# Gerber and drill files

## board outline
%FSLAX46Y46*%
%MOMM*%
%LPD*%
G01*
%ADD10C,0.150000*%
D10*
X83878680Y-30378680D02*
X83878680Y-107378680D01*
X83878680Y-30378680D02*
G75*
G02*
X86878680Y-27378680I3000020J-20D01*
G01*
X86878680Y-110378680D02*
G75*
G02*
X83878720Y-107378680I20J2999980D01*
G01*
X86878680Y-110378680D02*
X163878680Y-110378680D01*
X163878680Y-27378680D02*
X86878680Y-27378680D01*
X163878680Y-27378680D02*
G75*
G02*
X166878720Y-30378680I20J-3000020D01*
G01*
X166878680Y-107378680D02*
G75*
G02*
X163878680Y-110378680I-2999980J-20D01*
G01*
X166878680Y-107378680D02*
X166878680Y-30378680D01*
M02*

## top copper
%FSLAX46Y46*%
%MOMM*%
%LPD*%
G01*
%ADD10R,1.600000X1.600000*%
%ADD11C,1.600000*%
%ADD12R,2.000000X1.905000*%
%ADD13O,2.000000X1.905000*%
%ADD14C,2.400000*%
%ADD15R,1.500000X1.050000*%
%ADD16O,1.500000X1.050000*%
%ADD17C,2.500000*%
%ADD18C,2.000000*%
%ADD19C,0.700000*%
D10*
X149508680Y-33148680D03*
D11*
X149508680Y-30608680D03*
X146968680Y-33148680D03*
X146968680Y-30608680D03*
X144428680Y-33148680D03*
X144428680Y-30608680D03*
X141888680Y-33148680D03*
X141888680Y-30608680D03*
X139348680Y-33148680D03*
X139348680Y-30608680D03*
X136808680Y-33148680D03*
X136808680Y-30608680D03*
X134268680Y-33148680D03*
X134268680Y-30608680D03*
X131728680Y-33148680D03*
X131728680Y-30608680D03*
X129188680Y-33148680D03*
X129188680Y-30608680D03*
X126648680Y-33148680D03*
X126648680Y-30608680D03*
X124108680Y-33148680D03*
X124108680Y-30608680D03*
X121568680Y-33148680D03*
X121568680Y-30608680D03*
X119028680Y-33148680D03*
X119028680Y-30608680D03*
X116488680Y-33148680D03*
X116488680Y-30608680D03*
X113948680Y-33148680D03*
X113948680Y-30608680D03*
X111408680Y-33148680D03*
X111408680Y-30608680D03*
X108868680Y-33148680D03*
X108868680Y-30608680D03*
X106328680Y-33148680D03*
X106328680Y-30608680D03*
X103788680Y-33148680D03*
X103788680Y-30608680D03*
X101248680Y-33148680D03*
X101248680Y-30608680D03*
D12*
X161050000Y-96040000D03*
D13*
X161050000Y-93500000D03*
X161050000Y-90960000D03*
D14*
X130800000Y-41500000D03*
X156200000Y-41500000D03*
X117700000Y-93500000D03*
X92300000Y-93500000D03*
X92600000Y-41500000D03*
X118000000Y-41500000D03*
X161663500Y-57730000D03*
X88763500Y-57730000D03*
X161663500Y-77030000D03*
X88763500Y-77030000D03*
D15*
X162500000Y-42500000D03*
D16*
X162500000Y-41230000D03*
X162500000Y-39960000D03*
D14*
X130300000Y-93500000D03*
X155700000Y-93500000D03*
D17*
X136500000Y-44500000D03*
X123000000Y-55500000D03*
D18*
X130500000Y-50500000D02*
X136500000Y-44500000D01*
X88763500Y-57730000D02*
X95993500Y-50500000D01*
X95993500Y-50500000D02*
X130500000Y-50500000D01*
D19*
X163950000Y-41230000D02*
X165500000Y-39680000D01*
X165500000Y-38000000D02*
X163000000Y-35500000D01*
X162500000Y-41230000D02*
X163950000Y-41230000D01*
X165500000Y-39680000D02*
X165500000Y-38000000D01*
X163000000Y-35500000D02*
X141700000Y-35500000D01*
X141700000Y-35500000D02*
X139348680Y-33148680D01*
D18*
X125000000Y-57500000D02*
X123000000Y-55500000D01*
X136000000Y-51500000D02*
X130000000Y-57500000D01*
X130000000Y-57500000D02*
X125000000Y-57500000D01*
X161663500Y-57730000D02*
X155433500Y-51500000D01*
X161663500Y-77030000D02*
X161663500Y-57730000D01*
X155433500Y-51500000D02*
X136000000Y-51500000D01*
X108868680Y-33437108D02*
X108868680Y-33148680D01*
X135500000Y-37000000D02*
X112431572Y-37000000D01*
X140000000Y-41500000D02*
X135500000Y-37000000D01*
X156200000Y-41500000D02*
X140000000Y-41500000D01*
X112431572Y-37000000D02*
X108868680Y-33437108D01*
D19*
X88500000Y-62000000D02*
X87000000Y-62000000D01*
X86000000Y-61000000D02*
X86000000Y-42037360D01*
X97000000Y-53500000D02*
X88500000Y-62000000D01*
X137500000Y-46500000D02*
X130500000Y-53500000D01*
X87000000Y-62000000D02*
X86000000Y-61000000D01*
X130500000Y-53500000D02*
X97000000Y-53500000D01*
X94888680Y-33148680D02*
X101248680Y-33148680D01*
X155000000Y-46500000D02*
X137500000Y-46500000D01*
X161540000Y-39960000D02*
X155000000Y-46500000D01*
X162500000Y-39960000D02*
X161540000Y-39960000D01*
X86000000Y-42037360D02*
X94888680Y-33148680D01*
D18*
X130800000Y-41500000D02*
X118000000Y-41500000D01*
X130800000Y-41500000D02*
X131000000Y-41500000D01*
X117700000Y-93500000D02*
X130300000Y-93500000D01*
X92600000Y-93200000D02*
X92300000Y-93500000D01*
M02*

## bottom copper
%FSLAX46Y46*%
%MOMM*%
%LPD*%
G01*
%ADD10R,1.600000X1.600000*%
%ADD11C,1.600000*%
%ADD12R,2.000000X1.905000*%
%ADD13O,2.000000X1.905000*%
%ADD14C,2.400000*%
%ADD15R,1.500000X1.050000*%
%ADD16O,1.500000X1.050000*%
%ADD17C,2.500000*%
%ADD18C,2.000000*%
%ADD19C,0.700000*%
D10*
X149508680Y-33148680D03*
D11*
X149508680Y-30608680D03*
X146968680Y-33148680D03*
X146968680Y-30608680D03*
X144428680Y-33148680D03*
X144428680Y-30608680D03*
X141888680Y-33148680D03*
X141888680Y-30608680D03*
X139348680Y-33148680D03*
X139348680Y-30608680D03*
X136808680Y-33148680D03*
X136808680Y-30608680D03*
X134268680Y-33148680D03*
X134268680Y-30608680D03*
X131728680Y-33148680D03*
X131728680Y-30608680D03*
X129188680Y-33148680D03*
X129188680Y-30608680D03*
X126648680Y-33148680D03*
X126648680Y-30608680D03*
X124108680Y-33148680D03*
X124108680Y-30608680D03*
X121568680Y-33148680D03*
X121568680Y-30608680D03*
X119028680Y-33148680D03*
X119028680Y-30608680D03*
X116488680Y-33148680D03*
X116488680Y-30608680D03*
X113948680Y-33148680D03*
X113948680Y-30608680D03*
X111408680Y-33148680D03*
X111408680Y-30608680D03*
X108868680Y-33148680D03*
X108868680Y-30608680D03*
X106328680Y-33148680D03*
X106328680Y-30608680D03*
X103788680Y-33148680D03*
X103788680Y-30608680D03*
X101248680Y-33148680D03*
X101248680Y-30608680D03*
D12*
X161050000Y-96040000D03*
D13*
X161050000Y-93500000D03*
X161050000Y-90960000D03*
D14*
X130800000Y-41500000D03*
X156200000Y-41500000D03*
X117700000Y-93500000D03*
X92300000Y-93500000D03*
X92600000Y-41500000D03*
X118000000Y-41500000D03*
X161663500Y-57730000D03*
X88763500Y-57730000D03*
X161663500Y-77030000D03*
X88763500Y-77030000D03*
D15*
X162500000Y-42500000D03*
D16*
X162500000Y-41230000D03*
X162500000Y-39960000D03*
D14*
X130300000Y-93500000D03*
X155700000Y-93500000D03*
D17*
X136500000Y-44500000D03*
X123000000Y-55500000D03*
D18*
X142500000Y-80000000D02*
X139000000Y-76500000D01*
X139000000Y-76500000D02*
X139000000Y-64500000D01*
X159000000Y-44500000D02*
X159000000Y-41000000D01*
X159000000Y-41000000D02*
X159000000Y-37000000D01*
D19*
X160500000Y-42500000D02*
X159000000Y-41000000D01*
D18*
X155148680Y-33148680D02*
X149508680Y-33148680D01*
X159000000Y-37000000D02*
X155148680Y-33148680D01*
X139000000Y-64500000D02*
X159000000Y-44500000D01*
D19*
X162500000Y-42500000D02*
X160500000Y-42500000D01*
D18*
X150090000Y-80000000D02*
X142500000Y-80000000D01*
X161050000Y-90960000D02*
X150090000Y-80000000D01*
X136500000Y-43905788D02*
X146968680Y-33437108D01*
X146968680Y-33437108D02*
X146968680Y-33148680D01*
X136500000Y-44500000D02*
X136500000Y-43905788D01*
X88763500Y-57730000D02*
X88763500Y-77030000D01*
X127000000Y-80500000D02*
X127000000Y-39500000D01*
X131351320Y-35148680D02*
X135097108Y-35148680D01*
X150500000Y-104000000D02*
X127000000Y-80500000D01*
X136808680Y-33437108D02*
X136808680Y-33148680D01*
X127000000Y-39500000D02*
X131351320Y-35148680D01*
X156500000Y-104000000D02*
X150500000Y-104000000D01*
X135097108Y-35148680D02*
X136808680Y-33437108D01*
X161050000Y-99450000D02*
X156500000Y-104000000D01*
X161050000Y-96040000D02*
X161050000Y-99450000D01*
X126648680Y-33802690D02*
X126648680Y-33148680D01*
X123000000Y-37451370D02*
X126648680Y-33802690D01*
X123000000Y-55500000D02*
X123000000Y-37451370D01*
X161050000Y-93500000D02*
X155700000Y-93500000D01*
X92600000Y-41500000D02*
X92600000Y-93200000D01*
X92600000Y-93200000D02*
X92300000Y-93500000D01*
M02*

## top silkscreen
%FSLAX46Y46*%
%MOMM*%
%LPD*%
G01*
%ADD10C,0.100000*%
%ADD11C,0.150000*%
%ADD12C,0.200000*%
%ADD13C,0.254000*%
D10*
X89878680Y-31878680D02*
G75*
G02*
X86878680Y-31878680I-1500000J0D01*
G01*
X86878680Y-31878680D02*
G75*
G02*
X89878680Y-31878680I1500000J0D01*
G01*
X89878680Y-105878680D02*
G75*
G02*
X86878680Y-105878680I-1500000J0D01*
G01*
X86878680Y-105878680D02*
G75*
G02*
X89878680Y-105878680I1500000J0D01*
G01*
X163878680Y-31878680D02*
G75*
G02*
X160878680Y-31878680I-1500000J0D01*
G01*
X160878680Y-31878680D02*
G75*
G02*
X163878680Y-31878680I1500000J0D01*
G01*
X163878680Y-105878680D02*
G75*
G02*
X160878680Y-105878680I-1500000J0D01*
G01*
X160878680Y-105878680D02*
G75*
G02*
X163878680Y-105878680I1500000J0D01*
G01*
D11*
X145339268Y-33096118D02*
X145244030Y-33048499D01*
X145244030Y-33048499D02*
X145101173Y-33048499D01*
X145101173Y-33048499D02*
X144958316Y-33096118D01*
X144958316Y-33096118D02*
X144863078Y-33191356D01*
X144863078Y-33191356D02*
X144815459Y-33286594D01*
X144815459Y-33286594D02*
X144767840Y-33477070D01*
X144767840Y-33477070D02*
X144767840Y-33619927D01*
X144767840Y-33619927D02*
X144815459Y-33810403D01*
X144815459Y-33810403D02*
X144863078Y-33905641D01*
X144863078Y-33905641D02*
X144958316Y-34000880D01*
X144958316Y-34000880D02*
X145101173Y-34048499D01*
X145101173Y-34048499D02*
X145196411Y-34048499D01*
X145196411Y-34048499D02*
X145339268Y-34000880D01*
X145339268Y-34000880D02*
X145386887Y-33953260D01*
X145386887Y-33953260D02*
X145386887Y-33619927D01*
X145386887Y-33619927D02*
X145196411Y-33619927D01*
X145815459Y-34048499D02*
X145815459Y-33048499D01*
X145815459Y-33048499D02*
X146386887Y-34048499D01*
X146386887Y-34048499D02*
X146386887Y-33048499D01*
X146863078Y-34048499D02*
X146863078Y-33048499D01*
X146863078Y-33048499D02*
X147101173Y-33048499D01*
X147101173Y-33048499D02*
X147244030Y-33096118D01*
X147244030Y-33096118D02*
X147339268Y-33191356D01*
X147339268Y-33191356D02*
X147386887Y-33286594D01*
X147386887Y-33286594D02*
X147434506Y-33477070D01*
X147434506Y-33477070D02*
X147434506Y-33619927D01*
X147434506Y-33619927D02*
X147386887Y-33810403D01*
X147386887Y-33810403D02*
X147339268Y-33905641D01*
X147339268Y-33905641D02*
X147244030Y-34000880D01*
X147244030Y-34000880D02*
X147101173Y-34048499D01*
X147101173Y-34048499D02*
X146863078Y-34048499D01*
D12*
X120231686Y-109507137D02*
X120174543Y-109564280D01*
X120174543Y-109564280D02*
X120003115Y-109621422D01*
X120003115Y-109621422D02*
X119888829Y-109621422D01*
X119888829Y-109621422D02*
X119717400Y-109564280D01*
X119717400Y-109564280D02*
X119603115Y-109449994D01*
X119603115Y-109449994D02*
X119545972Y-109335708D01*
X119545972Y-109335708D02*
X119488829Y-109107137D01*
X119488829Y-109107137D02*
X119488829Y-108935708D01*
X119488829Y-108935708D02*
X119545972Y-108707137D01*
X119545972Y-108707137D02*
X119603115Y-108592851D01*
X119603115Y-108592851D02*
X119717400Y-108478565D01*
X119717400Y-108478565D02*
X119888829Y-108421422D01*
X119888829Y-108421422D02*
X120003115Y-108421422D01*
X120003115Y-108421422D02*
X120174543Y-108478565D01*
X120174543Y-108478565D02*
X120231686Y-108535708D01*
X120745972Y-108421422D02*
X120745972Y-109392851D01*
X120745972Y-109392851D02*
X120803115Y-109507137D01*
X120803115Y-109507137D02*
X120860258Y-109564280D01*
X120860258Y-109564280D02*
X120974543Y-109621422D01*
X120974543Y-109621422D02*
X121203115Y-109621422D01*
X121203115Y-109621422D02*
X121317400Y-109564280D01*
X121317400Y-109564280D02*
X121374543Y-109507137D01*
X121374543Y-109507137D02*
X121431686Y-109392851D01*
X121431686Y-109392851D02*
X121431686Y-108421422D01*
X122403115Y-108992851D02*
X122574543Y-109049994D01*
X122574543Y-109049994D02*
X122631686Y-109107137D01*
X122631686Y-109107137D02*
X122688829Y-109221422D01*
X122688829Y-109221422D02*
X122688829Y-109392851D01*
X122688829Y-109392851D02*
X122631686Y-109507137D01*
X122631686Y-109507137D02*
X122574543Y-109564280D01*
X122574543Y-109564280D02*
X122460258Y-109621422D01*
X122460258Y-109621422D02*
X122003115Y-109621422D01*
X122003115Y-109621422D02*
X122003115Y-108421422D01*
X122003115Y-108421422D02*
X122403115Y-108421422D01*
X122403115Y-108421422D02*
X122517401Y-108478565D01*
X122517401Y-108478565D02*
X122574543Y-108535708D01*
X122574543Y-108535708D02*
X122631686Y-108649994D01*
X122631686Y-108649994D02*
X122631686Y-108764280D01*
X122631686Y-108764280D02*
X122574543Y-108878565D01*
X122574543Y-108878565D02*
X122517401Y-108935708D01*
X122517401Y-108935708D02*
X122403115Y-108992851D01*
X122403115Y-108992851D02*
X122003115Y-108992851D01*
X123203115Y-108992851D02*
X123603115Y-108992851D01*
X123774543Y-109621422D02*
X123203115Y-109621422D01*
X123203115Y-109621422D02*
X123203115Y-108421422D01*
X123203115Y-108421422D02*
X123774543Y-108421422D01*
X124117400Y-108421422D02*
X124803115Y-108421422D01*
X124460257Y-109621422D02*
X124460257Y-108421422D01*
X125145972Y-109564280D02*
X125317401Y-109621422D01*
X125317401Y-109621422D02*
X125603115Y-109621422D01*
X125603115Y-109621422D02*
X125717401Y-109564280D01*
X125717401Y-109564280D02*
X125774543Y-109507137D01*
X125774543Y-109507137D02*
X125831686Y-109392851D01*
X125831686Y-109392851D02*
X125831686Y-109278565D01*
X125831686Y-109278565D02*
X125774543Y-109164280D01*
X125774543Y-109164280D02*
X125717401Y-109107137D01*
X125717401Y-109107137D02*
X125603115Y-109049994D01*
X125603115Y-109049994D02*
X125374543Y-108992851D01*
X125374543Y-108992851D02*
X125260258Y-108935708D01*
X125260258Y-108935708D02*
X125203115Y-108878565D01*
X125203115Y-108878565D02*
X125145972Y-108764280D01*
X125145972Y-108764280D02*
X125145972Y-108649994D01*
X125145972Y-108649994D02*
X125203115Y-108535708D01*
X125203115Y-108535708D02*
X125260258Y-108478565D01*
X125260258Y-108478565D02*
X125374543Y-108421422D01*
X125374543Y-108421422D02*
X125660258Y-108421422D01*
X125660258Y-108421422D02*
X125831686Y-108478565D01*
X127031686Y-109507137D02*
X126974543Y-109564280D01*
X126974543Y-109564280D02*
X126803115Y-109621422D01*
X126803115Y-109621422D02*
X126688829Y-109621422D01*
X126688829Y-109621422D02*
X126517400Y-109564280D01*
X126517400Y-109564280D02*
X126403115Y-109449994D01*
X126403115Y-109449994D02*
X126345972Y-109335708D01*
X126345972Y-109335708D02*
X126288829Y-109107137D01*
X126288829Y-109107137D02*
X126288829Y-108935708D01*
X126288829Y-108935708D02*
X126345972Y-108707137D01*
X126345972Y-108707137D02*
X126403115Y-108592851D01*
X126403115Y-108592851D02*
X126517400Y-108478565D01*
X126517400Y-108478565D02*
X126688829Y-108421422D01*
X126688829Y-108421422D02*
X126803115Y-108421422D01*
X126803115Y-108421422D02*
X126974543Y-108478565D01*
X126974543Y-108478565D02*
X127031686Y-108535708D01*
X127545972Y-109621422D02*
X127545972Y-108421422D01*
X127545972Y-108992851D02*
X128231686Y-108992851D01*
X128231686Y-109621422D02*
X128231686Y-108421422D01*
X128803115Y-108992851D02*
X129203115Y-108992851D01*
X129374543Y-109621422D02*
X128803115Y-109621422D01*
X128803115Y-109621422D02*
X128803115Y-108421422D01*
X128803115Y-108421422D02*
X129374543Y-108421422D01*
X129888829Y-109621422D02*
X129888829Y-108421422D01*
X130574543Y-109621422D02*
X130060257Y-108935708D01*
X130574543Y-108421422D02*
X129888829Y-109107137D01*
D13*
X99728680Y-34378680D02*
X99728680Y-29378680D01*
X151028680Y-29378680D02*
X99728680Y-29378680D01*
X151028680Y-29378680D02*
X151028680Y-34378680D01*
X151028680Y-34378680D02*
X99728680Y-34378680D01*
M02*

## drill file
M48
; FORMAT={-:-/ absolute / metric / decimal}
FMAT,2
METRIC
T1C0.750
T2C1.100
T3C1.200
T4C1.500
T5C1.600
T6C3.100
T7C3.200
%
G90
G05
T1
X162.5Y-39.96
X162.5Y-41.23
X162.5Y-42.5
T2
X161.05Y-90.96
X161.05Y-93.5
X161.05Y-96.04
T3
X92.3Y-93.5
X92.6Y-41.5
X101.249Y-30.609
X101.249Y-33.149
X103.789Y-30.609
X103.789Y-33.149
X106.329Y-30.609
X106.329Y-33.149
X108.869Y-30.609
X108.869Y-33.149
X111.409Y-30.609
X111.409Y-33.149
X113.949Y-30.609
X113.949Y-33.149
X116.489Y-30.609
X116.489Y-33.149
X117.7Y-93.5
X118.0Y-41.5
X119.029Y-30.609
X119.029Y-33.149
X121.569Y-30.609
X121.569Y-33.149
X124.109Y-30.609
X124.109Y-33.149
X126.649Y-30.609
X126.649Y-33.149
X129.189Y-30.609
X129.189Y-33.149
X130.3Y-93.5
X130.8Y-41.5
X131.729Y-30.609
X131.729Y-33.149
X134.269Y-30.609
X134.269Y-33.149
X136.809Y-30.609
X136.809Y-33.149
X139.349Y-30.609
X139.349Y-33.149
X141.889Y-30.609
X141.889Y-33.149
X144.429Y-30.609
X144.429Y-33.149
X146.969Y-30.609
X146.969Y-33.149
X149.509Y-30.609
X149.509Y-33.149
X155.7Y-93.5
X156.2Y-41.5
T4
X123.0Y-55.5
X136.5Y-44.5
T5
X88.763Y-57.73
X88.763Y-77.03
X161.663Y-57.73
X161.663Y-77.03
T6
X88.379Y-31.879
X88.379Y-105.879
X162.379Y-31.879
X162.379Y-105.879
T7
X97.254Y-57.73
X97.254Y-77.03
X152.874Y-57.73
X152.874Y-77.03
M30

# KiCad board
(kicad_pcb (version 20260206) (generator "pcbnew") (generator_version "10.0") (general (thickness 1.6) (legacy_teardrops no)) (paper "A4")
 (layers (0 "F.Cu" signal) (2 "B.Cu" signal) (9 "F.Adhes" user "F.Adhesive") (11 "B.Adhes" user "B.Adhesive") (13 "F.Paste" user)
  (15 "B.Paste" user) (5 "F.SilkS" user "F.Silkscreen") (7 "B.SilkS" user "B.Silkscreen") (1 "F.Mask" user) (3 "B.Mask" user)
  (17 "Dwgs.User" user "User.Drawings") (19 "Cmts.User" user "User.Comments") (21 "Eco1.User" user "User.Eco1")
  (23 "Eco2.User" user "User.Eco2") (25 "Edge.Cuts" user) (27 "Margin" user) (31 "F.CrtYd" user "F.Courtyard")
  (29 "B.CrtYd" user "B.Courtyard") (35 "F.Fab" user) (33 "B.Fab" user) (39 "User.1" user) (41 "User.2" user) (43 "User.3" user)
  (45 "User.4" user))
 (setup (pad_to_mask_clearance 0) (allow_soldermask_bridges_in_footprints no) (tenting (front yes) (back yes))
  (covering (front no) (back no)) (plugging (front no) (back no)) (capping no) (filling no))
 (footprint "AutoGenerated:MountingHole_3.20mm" (layer "F.Cu") (at 88.37868 105.87868)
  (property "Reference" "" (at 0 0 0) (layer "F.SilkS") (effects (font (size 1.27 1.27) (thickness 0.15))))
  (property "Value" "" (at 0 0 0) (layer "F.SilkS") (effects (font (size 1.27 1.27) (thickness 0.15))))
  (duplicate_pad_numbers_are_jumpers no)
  (pad "" np_thru_hole circle (at 0 0) (size 3.1 3.1) (drill 3.1) (layers "*.Cu" "*.Mask")))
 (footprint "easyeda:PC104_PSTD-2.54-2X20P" (layer "F.Cu") (at 149.50868 30.60868 -90)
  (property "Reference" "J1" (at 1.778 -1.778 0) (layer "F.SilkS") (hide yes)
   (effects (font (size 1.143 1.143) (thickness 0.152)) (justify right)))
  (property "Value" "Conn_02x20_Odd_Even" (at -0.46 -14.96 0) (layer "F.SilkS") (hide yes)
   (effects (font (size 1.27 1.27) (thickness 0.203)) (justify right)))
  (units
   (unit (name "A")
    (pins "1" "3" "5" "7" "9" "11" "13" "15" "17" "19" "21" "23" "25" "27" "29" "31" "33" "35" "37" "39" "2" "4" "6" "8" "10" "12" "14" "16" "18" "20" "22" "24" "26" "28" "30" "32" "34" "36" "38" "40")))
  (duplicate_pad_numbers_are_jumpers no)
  (fp_line (start 3.77 49.78) (end -1.23 49.78) (stroke (width 0.254) (type solid)) (layer "F.SilkS"))
  (fp_line (start -1.23 -1.52) (end -1.23 49.78) (stroke (width 0.254) (type solid)) (layer "F.SilkS"))
  (fp_line (start -1.23 -1.52) (end 3.77 -1.52) (stroke (width 0.254) (type solid)) (layer "F.SilkS"))
  (fp_line (start 3.77 -1.52) (end 3.77 49.78) (stroke (width 0.254) (type solid)) (layer "F.SilkS"))
  (pad "1" thru_hole rect (at 2.54 0 180) (size 1.6 1.6) (drill 1.2) (layers "*.Cu" "*.Paste" "*.Mask") (remove_unused_layers no)
   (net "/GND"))
  (pad "2" thru_hole circle (at 0 0 180) (size 1.6 1.6) (drill 1.2) (layers "*.Cu" "*.Paste" "*.Mask") (remove_unused_layers no)
   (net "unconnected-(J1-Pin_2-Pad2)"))
  (pad "3" thru_hole circle (at 2.54 2.54 180) (size 1.6 1.6) (drill 1.2) (layers "*.Cu" "*.Paste" "*.Mask") (remove_unused_layers no)
   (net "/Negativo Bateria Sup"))
  (pad "4" thru_hole circle (at 0 2.54 180) (size 1.6 1.6) (drill 1.2) (layers "*.Cu" "*.Paste" "*.Mask") (remove_unused_layers no)
   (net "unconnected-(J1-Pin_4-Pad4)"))
  (pad "5" thru_hole circle (at 2.54 5.08 180) (size 1.6 1.6) (drill 1.2) (layers "*.Cu" "*.Paste" "*.Mask") (remove_unused_layers no)
   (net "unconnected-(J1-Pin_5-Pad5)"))
  (pad "6" thru_hole circle (at 0 5.08 180) (size 1.6 1.6) (drill 1.2) (layers "*.Cu" "*.Paste" "*.Mask") (remove_unused_layers no)
   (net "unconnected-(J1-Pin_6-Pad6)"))
  (pad "7" thru_hole circle (at 2.54 7.62 180) (size 1.6 1.6) (drill 1.2) (layers "*.Cu" "*.Paste" "*.Mask") (remove_unused_layers no)
   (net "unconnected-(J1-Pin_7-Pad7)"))
  (pad "8" thru_hole circle (at 0 7.62 180) (size 1.6 1.6) (drill 1.2) (layers "*.Cu" "*.Paste" "*.Mask") (remove_unused_layers no)
   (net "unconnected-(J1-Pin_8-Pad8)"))
  (pad "9" thru_hole circle (at 2.54 10.16 180) (size 1.6 1.6) (drill 1.2) (layers "*.Cu" "*.Paste" "*.Mask") (remove_unused_layers no)
   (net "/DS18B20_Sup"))
  (pad "10" thru_hole circle (at 0 10.16 180) (size 1.6 1.6) (drill 1.2) (layers "*.Cu" "*.Paste" "*.Mask") (remove_unused_layers no)
   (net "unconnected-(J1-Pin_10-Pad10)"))
  (pad "11" thru_hole circle (at 2.54 12.7 180) (size 1.6 1.6) (drill 1.2) (layers "*.Cu" "*.Paste" "*.Mask") (remove_unused_layers no)
   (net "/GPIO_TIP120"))
  (pad "12" thru_hole circle (at 0 12.7 180) (size 1.6 1.6) (drill 1.2) (layers "*.Cu" "*.Paste" "*.Mask") (remove_unused_layers no)
   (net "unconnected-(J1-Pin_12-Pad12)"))
  (pad "13" thru_hole circle (at 2.54 15.24 180) (size 1.6 1.6) (drill 1.2) (layers "*.Cu" "*.Paste" "*.Mask") (remove_unused_layers no)
   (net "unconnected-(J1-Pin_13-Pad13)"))
  (pad "14" thru_hole circle (at 0 15.24 180) (size 1.6 1.6) (drill 1.2) (layers "*.Cu" "*.Paste" "*.Mask") (remove_unused_layers no)
   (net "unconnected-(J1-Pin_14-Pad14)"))
  (pad "15" thru_hole circle (at 2.54 17.78 180) (size 1.6 1.6) (drill 1.2) (layers "*.Cu" "*.Paste" "*.Mask") (remove_unused_layers no)
   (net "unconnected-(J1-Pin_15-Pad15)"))
  (pad "16" thru_hole circle (at 0 17.78 180) (size 1.6 1.6) (drill 1.2) (layers "*.Cu" "*.Paste" "*.Mask") (remove_unused_layers no)
   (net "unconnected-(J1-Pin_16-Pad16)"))
  (pad "17" thru_hole circle (at 2.54 20.32 180) (size 1.6 1.6) (drill 1.2) (layers "*.Cu" "*.Paste" "*.Mask") (remove_unused_layers no)
   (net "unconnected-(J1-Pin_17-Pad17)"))
  (pad "18" thru_hole circle (at 0 20.32 180) (size 1.6 1.6) (drill 1.2) (layers "*.Cu" "*.Paste" "*.Mask") (remove_unused_layers no)
   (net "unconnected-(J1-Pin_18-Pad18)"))
  (pad "19" thru_hole circle (at 2.54 22.86 180) (size 1.6 1.6) (drill 1.2) (layers "*.Cu" "*.Paste" "*.Mask") (remove_unused_layers no)
   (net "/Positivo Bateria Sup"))
  (pad "20" thru_hole circle (at 0 22.86 180) (size 1.6 1.6) (drill 1.2) (layers "*.Cu" "*.Paste" "*.Mask") (remove_unused_layers no)
   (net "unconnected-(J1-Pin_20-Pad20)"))
  (pad "21" thru_hole circle (at 2.54 25.4 180) (size 1.6 1.6) (drill 1.2) (layers "*.Cu" "*.Paste" "*.Mask") (remove_unused_layers no)
   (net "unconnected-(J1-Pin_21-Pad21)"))
  (pad "22" thru_hole circle (at 0 25.4 180) (size 1.6 1.6) (drill 1.2) (layers "*.Cu" "*.Paste" "*.Mask") (remove_unused_layers no)
   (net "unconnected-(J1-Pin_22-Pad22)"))
  (pad "23" thru_hole circle (at 2.54 27.94 180) (size 1.6 1.6) (drill 1.2) (layers "*.Cu" "*.Paste" "*.Mask") (remove_unused_layers no)
   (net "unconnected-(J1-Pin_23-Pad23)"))
  (pad "24" thru_hole circle (at 0 27.94 180) (size 1.6 1.6) (drill 1.2) (layers "*.Cu" "*.Paste" "*.Mask") (remove_unused_layers no)
   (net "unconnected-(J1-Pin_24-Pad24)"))
  (pad "25" thru_hole circle (at 2.54 30.48 180) (size 1.6 1.6) (drill 1.2) (layers "*.Cu" "*.Paste" "*.Mask") (remove_unused_layers no)
   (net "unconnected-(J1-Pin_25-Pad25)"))
  (pad "26" thru_hole circle (at 0 30.48 180) (size 1.6 1.6) (drill 1.2) (layers "*.Cu" "*.Paste" "*.Mask") (remove_unused_layers no)
   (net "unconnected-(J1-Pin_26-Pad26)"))
  (pad "27" thru_hole circle (at 2.54 33.02 180) (size 1.6 1.6) (drill 1.2) (layers "*.Cu" "*.Paste" "*.Mask") (remove_unused_layers no)
   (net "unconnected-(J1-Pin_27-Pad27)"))
  (pad "28" thru_hole circle (at 0 33.02 180) (size 1.6 1.6) (drill 1.2) (layers "*.Cu" "*.Paste" "*.Mask") (remove_unused_layers no)
   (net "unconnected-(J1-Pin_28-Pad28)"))
  (pad "29" thru_hole circle (at 2.54 35.56 180) (size 1.6 1.6) (drill 1.2) (layers "*.Cu" "*.Paste" "*.Mask") (remove_unused_layers no)
   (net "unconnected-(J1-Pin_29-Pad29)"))
  (pad "30" thru_hole circle (at 0 35.56 180) (size 1.6 1.6) (drill 1.2) (layers "*.Cu" "*.Paste" "*.Mask") (remove_unused_layers no)
   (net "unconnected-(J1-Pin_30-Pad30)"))
  (pad "31" thru_hole circle (at 2.54 38.1 180) (size 1.6 1.6) (drill 1.2) (layers "*.Cu" "*.Paste" "*.Mask") (remove_unused_layers no)
   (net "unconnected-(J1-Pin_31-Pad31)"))
  (pad "32" thru_hole circle (at 0 38.1 180) (size 1.6 1.6) (drill 1.2) (layers "*.Cu" "*.Paste" "*.Mask") (remove_unused_layers no)
   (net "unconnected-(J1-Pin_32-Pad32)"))
  (pad "33" thru_hole circle (at 2.54 40.64 180) (size 1.6 1.6) (drill 1.2) (layers "*.Cu" "*.Paste" "*.Mask") (remove_unused_layers no)
   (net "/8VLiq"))
  (pad "34" thru_hole circle (at 0 40.64 180) (size 1.6 1.6) (drill 1.2) (layers "*.Cu" "*.Paste" "*.Mask") (remove_unused_layers no)
   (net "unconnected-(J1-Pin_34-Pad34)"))
  (pad "35" thru_hole circle (at 2.54 43.18 180) (size 1.6 1.6) (drill 1.2) (layers "*.Cu" "*.Paste" "*.Mask") (remove_unused_layers no)
   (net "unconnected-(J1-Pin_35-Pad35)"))
  (pad "36" thru_hole circle (at 0 43.18 180) (size 1.6 1.6) (drill 1.2) (layers "*.Cu" "*.Paste" "*.Mask") (remove_unused_layers no)
   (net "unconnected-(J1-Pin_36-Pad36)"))
  (pad "37" thru_hole circle (at 2.54 45.72 180) (size 1.6 1.6) (drill 1.2) (layers "*.Cu" "*.Paste" "*.Mask") (remove_unused_layers no)
   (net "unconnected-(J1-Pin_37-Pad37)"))
  (pad "38" thru_hole circle (at 0 45.72 180) (size 1.6 1.6) (drill 1.2) (layers "*.Cu" "*.Paste" "*.Mask") (remove_unused_layers no)
   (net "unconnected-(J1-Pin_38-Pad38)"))
  (pad "39" thru_hole circle (at 2.54 48.26 180) (size 1.6 1.6) (drill 1.2) (layers "*.Cu" "*.Paste" "*.Mask") (remove_unused_layers no)
   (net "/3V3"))
  (pad "40" thru_hole circle (at 0 48.26 180) (size 1.6 1.6) (drill 1.2) (layers "*.Cu" "*.Paste" "*.Mask") (remove_unused_layers no)
   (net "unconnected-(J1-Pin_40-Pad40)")))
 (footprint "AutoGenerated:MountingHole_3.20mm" (layer "F.Cu") (at 88.37868 31.87868)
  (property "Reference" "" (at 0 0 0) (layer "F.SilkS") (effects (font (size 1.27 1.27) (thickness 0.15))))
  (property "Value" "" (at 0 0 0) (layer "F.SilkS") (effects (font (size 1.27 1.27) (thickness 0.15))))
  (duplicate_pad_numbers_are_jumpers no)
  (pad "" np_thru_hole circle (at 0 0) (size 3.1 3.1) (drill 3.1) (layers "*.Cu" "*.Mask")))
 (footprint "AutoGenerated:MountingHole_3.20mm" (layer "F.Cu") (at 162.37868 31.87868)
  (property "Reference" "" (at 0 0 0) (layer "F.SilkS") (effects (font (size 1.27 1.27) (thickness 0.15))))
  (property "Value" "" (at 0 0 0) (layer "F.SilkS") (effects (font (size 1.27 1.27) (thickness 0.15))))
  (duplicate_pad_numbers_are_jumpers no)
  (pad "" np_thru_hole circle (at 0 0) (size 3.1 3.1) (drill 3.1) (layers "*.Cu" "*.Mask")))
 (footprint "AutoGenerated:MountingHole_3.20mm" (layer "F.Cu") (at 162.37868 105.87868)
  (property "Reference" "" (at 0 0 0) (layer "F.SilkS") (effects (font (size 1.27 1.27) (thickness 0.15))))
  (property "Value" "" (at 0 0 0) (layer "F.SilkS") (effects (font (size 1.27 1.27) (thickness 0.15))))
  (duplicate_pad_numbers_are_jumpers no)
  (pad "" np_thru_hole circle (at 0 0) (size 3.1 3.1) (drill 3.1) (layers "*.Cu" "*.Mask")))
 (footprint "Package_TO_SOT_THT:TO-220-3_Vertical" (layer "B.Cu") (at 161.05 96.04 90)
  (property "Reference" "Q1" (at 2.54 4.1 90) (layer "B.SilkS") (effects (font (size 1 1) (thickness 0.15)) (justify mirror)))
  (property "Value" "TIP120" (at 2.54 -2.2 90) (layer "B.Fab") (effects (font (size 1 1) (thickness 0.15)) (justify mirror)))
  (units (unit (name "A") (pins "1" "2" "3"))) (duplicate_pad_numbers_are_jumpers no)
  (pad "1" thru_hole rect (at 0 0 90) (size 1.905 2) (drill 1.1) (layers "*.Cu" "*.Mask") (remove_unused_layers no) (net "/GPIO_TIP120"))
  (pad "2" thru_hole oval (at 2.54 0 90) (size 1.905 2) (drill 1.1) (layers "*.Cu" "*.Mask") (remove_unused_layers no) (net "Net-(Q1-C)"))
  (pad "3" thru_hole oval (at 5.08 0 90) (size 1.905 2) (drill 1.1) (layers "*.Cu" "*.Mask") (remove_unused_layers no) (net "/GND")))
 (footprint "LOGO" (layer "B.Cu") (at 155.04 108.58 180)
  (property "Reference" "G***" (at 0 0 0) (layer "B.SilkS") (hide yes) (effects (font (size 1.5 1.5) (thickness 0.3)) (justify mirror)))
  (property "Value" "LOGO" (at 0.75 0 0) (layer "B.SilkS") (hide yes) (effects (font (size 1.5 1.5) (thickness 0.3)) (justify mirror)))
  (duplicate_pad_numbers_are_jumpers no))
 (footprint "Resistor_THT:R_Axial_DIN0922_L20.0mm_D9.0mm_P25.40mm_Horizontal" (layer "B.Cu") (at 130.8 41.5)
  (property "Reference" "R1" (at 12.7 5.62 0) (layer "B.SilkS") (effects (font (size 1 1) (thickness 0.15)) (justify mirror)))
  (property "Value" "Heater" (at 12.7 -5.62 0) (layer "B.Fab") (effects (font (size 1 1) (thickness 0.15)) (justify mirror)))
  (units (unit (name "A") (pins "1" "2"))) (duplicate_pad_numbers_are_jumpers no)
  (pad "1" thru_hole circle (at 0 0) (size 2.4 2.4) (drill 1.2) (layers "*.Cu" "*.Mask") (remove_unused_layers no) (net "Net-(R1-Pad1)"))
  (pad "2" thru_hole circle (at 25.4 0) (size 2.4 2.4) (drill 1.2) (layers "*.Cu" "*.Mask") (remove_unused_layers no) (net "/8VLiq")))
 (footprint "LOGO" (layer "B.Cu") (at 141.48 106.05 90)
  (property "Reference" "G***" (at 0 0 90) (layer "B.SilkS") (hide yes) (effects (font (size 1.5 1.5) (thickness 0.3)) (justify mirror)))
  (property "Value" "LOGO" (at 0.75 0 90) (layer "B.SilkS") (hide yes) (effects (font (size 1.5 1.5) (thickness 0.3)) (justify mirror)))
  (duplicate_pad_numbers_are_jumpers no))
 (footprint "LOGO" (layer "B.Cu") (at 95.42 108.6 180)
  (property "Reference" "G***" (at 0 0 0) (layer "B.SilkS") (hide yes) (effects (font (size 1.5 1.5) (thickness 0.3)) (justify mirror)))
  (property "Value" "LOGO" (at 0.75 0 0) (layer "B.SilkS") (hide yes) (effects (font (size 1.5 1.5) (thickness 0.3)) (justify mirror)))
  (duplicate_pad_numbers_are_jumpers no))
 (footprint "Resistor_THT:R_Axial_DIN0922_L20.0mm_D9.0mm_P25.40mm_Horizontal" (layer "B.Cu") (at 117.7 93.5 180)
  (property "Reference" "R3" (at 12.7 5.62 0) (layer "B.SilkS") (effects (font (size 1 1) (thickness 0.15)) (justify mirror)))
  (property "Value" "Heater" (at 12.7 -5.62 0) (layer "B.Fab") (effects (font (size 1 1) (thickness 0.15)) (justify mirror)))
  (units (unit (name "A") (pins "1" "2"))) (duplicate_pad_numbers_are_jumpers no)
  (pad "1" thru_hole circle (at 0 0 180) (size 2.4 2.4) (drill 1.2) (layers "*.Cu" "*.Mask") (remove_unused_layers no) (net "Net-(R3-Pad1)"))
  (pad "2" thru_hole circle (at 25.4 0 180) (size 2.4 2.4) (drill 1.2) (layers "*.Cu" "*.Mask") (remove_unused_layers no)
   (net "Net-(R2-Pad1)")))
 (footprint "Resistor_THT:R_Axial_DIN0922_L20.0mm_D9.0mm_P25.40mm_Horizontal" (layer "B.Cu") (at 92.6 41.5)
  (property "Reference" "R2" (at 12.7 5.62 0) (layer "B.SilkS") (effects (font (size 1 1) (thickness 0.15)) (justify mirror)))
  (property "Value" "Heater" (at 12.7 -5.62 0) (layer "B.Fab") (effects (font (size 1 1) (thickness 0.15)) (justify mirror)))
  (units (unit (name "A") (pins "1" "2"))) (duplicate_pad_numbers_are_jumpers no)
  (pad "1" thru_hole circle (at 0 0) (size 2.4 2.4) (drill 1.2) (layers "*.Cu" "*.Mask") (remove_unused_layers no) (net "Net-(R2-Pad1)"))
  (pad "2" thru_hole circle (at 25.4 0) (size 2.4 2.4) (drill 1.2) (layers "*.Cu" "*.Mask") (remove_unused_layers no) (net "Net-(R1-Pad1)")))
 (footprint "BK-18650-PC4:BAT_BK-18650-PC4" (layer "B.Cu") (at 125.0635 67.38 180)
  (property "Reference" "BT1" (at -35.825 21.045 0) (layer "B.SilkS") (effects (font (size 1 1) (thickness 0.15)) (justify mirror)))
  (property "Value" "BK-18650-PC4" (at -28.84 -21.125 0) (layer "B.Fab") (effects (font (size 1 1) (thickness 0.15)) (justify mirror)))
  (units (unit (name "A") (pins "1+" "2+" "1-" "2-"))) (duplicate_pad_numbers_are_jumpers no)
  (pad "" np_thru_hole circle (at -27.81 -9.65 180) (size 3.2 3.2) (drill 3.2) (layers "*.Cu" "*.Mask"))
  (pad "" np_thru_hole circle (at -27.81 9.65 180) (size 3.2 3.2) (drill 3.2) (layers "*.Cu" "*.Mask"))
  (pad "" np_thru_hole circle (at 27.81 -9.65 180) (size 3.2 3.2) (drill 3.2) (layers "*.Cu" "*.Mask"))
  (pad "" np_thru_hole circle (at 27.81 9.65 180) (size 3.2 3.2) (drill 3.2) (layers "*.Cu" "*.Mask"))
  (pad "1+" thru_hole circle (at -36.6 9.65 180) (size 2.4 2.4) (drill 1.6) (layers "*.Cu" "*.Mask") (remove_unused_layers no)
   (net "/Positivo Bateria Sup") (solder_mask_margin 0.102))
  (pad "1-" thru_hole circle (at 36.3 9.65 180) (size 2.4 2.4) (drill 1.6) (layers "*.Cu" "*.Mask") (remove_unused_layers no)
   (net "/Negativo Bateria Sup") (solder_mask_margin 0.102))
  (pad "2+" thru_hole circle (at -36.6 -9.65 180) (size 2.4 2.4) (drill 1.6) (layers "*.Cu" "*.Mask") (remove_unused_layers no)
   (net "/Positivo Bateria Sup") (solder_mask_margin 0.102))
  (pad "2-" thru_hole circle (at 36.3 -9.65 180) (size 2.4 2.4) (drill 1.6) (layers "*.Cu" "*.Mask") (remove_unused_layers no)
   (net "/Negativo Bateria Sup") (solder_mask_margin 0.102)))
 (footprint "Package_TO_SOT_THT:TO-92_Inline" (layer "B.Cu") (at 162.5 42.5 90)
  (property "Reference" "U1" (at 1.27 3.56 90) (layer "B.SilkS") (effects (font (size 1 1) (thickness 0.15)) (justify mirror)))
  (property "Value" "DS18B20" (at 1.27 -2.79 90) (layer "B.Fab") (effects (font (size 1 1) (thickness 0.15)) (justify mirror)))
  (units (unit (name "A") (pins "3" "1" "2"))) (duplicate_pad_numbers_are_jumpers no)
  (pad "1" thru_hole rect (at 0 0 90) (size 1.05 1.5) (drill 0.75) (layers "*.Cu" "*.Mask") (remove_unused_layers no) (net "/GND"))
  (pad "2" thru_hole oval (at 1.27 0 90) (size 1.05 1.5) (drill 0.75) (layers "*.Cu" "*.Mask") (remove_unused_layers no)
   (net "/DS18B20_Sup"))
  (pad "3" thru_hole oval (at 2.54 0 90) (size 1.05 1.5) (drill 0.75) (layers "*.Cu" "*.Mask") (remove_unused_layers no) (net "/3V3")))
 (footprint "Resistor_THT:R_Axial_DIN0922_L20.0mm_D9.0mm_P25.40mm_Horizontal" (layer "B.Cu") (at 130.3 93.5)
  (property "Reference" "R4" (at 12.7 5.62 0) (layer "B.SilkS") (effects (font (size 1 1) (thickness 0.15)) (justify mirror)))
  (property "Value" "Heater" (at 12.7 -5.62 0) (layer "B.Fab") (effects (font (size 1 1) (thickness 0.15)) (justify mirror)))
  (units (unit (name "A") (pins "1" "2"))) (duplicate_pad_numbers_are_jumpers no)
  (pad "1" thru_hole circle (at 0 0) (size 2.4 2.4) (drill 1.2) (layers "*.Cu" "*.Mask") (remove_unused_layers no) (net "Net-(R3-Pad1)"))
  (pad "2" thru_hole circle (at 25.4 0) (size 2.4 2.4) (drill 1.2) (layers "*.Cu" "*.Mask") (remove_unused_layers no) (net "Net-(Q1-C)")))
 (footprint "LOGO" (layer "B.Cu") (at 106.21 106.15 180)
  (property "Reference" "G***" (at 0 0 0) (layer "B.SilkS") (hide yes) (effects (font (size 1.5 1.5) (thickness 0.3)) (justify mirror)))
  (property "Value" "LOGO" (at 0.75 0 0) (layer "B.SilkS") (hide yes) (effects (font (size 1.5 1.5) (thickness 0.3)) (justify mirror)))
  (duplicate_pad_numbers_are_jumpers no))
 (gr_circle (center 88.37868 31.87868) (end 89.87868 31.87868) (stroke (width 0.1) (type solid)) (fill no) (layer "F.SilkS"))
 (gr_circle (center 88.37868 105.87868) (end 89.87868 105.87868) (stroke (width 0.1) (type solid)) (fill no) (layer "F.SilkS"))
 (gr_circle (center 162.37868 31.87868) (end 163.87868 31.87868) (stroke (width 0.1) (type solid)) (fill no) (layer "F.SilkS"))
 (gr_circle (center 162.37868 105.87868) (end 163.87868 105.87868) (stroke (width 0.1) (type default)) (fill no) (layer "F.SilkS"))
 (gr_line (start 83.87868 30.37868) (end 83.87868 107.37868) (stroke (width 0.15) (type solid)) (layer "Edge.Cuts"))
 (gr_arc (start 83.87868 30.37868) (mid 84.75736 28.25736) (end 86.87868 27.37868) (stroke (width 0.15) (type solid)) (layer "Edge.Cuts"))
 (gr_arc (start 86.87868 110.37868) (mid 84.75736 109.5) (end 83.87868 107.37868) (stroke (width 0.15) (type solid)) (layer "Edge.Cuts"))
 (gr_line (start 86.87868 110.37868) (end 163.87868 110.37868) (stroke (width 0.15) (type solid)) (layer "Edge.Cuts"))
 (gr_line (start 163.87868 27.37868) (end 86.87868 27.37868) (stroke (width 0.15) (type solid)) (layer "Edge.Cuts"))
 (gr_arc (start 163.87868 27.37868) (mid 166 28.25736) (end 166.87868 30.37868) (stroke (width 0.15) (type solid)) (layer "Edge.Cuts"))
 (gr_arc (start 166.87868 107.37868) (mid 166 109.5) (end 163.87868 110.37868) (stroke (width 0.15) (type solid)) (layer "Edge.Cuts"))
 (gr_line (start 166.87868 107.37868) (end 166.87868 30.37868) (stroke (width 0.15) (type solid)) (layer "Edge.Cuts"))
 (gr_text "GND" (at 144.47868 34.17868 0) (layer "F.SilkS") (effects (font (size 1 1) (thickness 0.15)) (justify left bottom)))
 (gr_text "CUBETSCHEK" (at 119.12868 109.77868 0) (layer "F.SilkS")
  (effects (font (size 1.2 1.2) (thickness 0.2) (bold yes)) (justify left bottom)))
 (segment (start 142.5 80) (end 139 76.5) (width 2) (layer "B.Cu") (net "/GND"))
 (segment (start 139 76.5) (end 139 64.5) (width 2) (layer "B.Cu") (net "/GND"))
 (segment (start 159 44.5) (end 159 41) (width 2) (layer "B.Cu") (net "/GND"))
 (segment (start 159 41) (end 159 37) (width 2) (layer "B.Cu") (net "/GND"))
 (segment (start 160.5 42.5) (end 159 41) (width 0.7) (layer "B.Cu") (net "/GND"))
 (segment (start 155.14868 33.14868) (end 149.50868 33.14868) (width 2) (layer "B.Cu") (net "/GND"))
 (segment (start 159 37) (end 155.14868 33.14868) (width 2) (layer "B.Cu") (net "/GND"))
 (segment (start 139 64.5) (end 159 44.5) (width 2) (layer "B.Cu") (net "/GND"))
 (segment (start 162.5 42.5) (end 160.5 42.5) (width 0.7) (layer "B.Cu") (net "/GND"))
 (segment (start 150.09 80) (end 142.5 80) (width 2) (layer "B.Cu") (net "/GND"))
 (segment (start 161.05 90.96) (end 150.09 80) (width 2) (layer "B.Cu") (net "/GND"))
 (segment (start 130.5 50.5) (end 136.5 44.5) (width 2) (layer "F.Cu") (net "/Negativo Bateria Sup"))
 (segment (start 88.7635 57.73) (end 95.9935 50.5) (width 2) (layer "F.Cu") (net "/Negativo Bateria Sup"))
 (segment (start 95.9935 50.5) (end 130.5 50.5) (width 2) (layer "F.Cu") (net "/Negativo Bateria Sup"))
 (via (at 136.5 44.5) (size 2.5) (drill 1.5) (layers "F.Cu" "B.Cu") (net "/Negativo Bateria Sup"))
 (segment (start 136.5 43.905788) (end 146.96868 33.437108) (width 2) (layer "B.Cu") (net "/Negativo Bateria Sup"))
 (segment (start 146.96868 33.437108) (end 146.96868 33.14868) (width 2) (layer "B.Cu") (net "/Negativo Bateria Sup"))
 (segment (start 136.5 44.5) (end 136.5 43.905788) (width 2) (layer "B.Cu") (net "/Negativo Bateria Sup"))
 (segment (start 88.7635 57.73) (end 88.7635 77.03) (width 2) (layer "B.Cu") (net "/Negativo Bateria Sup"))
 (segment (start 163.95 41.23) (end 165.5 39.68) (width 0.7) (layer "F.Cu") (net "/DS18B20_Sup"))
 (segment (start 165.5 38) (end 163 35.5) (width 0.7) (layer "F.Cu") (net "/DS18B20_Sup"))
 (segment (start 162.5 41.23) (end 163.95 41.23) (width 0.7) (layer "F.Cu") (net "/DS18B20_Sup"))
 (segment (start 165.5 39.68) (end 165.5 38) (width 0.7) (layer "F.Cu") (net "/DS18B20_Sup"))
 (segment (start 163 35.5) (end 141.7 35.5) (width 0.7) (layer "F.Cu") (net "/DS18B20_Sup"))
 (segment (start 141.7 35.5) (end 139.34868 33.14868) (width 0.7) (layer "F.Cu") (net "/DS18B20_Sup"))
 (segment (start 127 80.5) (end 127 39.5) (width 2) (layer "B.Cu") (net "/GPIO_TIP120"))
 (segment (start 131.35132 35.14868) (end 135.097108 35.14868) (width 2) (layer "B.Cu") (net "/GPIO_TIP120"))
 (segment (start 150.5 104) (end 127 80.5) (width 2) (layer "B.Cu") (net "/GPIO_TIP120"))
 (segment (start 136.80868 33.437108) (end 136.80868 33.14868) (width 2) (layer "B.Cu") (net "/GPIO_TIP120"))
 (segment (start 127 39.5) (end 131.35132 35.14868) (width 2) (layer "B.Cu") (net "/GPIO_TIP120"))
 (segment (start 156.5 104) (end 150.5 104) (width 2) (layer "B.Cu") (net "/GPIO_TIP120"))
 (segment (start 135.097108 35.14868) (end 136.80868 33.437108) (width 2) (layer "B.Cu") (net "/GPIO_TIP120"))
 (segment (start 161.05 99.45) (end 156.5 104) (width 2) (layer "B.Cu") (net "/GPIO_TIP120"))
 (segment (start 161.05 96.04) (end 161.05 99.45) (width 2) (layer "B.Cu") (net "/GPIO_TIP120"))
 (segment (start 125 57.5) (end 123 55.5) (width 2) (layer "F.Cu") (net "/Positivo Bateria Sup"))
 (segment (start 136 51.5) (end 130 57.5) (width 2) (layer "F.Cu") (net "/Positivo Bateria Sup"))
 (segment (start 130 57.5) (end 125 57.5) (width 2) (layer "F.Cu") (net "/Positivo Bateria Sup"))
 (segment (start 161.6635 57.73) (end 155.4335 51.5) (width 2) (layer "F.Cu") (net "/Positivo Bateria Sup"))
 (segment (start 161.6635 77.03) (end 161.6635 57.73) (width 2) (layer "F.Cu") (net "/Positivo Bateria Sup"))
 (segment (start 155.4335 51.5) (end 136 51.5) (width 2) (layer "F.Cu") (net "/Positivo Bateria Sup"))
 (via (at 123 55.5) (size 2.5) (drill 1.5) (layers "F.Cu" "B.Cu") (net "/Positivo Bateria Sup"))
 (segment (start 126.64868 33.80269) (end 126.64868 33.14868) (width 2) (layer "B.Cu") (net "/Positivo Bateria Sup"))
 (segment (start 123 37.45137) (end 126.64868 33.80269) (width 2) (layer "B.Cu") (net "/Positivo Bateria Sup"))
 (segment (start 123 55.5) (end 123 37.45137) (width 2) (layer "B.Cu") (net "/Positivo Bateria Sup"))
 (segment (start 108.86868 33.437108) (end 108.86868 33.14868) (width 2) (layer "F.Cu") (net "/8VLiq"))
 (segment (start 135.5 37) (end 112.431572 37) (width 2) (layer "F.Cu") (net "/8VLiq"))
 (segment (start 140 41.5) (end 135.5 37) (width 2) (layer "F.Cu") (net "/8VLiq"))
 (segment (start 156.2 41.5) (end 140 41.5) (width 2) (layer "F.Cu") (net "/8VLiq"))
 (segment (start 112.431572 37) (end 108.86868 33.437108) (width 2) (layer "F.Cu") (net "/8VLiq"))
 (segment (start 88.5 62) (end 87 62) (width 0.7) (layer "F.Cu") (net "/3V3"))
 (segment (start 86 61) (end 86 42.03736) (width 0.7) (layer "F.Cu") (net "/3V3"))
 (segment (start 97 53.5) (end 88.5 62) (width 0.7) (layer "F.Cu") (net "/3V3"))
 (segment (start 137.5 46.5) (end 130.5 53.5) (width 0.7) (layer "F.Cu") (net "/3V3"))
 (segment (start 87 62) (end 86 61) (width 0.7) (layer "F.Cu") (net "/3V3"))
 (segment (start 130.5 53.5) (end 97 53.5) (width 0.7) (layer "F.Cu") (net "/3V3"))
 (segment (start 94.88868 33.14868) (end 101.24868 33.14868) (width 0.7) (layer "F.Cu") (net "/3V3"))
 (segment (start 155 46.5) (end 137.5 46.5) (width 0.7) (layer "F.Cu") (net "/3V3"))
 (segment (start 161.54 39.96) (end 155 46.5) (width 0.7) (layer "F.Cu") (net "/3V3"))
 (segment (start 162.5 39.96) (end 161.54 39.96) (width 0.7) (layer "F.Cu") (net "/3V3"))
 (segment (start 86 42.03736) (end 94.88868 33.14868) (width 0.7) (layer "F.Cu") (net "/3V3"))
 (segment (start 161.05 93.5) (end 155.7 93.5) (width 2) (layer "B.Cu") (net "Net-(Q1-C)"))
 (segment (start 130.8 41.5) (end 118 41.5) (width 2) (layer "F.Cu") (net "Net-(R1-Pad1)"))
 (segment (start 130.8 41.5) (end 131 41.5) (width 2) (layer "F.Cu") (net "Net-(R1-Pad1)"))
 (segment (start 117.7 93.5) (end 130.3 93.5) (width 2) (layer "F.Cu") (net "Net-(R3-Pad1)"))
 (segment (start 92.6 93.2) (end 92.3 93.5) (width 2) (layer "F.Cu") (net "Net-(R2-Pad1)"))
 (segment (start 92.6 41.5) (end 92.6 93.2) (width 2) (layer "B.Cu") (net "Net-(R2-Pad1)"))
 (segment (start 92.6 93.2) (end 92.3 93.5) (width 2) (layer "B.Cu") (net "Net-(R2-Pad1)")))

